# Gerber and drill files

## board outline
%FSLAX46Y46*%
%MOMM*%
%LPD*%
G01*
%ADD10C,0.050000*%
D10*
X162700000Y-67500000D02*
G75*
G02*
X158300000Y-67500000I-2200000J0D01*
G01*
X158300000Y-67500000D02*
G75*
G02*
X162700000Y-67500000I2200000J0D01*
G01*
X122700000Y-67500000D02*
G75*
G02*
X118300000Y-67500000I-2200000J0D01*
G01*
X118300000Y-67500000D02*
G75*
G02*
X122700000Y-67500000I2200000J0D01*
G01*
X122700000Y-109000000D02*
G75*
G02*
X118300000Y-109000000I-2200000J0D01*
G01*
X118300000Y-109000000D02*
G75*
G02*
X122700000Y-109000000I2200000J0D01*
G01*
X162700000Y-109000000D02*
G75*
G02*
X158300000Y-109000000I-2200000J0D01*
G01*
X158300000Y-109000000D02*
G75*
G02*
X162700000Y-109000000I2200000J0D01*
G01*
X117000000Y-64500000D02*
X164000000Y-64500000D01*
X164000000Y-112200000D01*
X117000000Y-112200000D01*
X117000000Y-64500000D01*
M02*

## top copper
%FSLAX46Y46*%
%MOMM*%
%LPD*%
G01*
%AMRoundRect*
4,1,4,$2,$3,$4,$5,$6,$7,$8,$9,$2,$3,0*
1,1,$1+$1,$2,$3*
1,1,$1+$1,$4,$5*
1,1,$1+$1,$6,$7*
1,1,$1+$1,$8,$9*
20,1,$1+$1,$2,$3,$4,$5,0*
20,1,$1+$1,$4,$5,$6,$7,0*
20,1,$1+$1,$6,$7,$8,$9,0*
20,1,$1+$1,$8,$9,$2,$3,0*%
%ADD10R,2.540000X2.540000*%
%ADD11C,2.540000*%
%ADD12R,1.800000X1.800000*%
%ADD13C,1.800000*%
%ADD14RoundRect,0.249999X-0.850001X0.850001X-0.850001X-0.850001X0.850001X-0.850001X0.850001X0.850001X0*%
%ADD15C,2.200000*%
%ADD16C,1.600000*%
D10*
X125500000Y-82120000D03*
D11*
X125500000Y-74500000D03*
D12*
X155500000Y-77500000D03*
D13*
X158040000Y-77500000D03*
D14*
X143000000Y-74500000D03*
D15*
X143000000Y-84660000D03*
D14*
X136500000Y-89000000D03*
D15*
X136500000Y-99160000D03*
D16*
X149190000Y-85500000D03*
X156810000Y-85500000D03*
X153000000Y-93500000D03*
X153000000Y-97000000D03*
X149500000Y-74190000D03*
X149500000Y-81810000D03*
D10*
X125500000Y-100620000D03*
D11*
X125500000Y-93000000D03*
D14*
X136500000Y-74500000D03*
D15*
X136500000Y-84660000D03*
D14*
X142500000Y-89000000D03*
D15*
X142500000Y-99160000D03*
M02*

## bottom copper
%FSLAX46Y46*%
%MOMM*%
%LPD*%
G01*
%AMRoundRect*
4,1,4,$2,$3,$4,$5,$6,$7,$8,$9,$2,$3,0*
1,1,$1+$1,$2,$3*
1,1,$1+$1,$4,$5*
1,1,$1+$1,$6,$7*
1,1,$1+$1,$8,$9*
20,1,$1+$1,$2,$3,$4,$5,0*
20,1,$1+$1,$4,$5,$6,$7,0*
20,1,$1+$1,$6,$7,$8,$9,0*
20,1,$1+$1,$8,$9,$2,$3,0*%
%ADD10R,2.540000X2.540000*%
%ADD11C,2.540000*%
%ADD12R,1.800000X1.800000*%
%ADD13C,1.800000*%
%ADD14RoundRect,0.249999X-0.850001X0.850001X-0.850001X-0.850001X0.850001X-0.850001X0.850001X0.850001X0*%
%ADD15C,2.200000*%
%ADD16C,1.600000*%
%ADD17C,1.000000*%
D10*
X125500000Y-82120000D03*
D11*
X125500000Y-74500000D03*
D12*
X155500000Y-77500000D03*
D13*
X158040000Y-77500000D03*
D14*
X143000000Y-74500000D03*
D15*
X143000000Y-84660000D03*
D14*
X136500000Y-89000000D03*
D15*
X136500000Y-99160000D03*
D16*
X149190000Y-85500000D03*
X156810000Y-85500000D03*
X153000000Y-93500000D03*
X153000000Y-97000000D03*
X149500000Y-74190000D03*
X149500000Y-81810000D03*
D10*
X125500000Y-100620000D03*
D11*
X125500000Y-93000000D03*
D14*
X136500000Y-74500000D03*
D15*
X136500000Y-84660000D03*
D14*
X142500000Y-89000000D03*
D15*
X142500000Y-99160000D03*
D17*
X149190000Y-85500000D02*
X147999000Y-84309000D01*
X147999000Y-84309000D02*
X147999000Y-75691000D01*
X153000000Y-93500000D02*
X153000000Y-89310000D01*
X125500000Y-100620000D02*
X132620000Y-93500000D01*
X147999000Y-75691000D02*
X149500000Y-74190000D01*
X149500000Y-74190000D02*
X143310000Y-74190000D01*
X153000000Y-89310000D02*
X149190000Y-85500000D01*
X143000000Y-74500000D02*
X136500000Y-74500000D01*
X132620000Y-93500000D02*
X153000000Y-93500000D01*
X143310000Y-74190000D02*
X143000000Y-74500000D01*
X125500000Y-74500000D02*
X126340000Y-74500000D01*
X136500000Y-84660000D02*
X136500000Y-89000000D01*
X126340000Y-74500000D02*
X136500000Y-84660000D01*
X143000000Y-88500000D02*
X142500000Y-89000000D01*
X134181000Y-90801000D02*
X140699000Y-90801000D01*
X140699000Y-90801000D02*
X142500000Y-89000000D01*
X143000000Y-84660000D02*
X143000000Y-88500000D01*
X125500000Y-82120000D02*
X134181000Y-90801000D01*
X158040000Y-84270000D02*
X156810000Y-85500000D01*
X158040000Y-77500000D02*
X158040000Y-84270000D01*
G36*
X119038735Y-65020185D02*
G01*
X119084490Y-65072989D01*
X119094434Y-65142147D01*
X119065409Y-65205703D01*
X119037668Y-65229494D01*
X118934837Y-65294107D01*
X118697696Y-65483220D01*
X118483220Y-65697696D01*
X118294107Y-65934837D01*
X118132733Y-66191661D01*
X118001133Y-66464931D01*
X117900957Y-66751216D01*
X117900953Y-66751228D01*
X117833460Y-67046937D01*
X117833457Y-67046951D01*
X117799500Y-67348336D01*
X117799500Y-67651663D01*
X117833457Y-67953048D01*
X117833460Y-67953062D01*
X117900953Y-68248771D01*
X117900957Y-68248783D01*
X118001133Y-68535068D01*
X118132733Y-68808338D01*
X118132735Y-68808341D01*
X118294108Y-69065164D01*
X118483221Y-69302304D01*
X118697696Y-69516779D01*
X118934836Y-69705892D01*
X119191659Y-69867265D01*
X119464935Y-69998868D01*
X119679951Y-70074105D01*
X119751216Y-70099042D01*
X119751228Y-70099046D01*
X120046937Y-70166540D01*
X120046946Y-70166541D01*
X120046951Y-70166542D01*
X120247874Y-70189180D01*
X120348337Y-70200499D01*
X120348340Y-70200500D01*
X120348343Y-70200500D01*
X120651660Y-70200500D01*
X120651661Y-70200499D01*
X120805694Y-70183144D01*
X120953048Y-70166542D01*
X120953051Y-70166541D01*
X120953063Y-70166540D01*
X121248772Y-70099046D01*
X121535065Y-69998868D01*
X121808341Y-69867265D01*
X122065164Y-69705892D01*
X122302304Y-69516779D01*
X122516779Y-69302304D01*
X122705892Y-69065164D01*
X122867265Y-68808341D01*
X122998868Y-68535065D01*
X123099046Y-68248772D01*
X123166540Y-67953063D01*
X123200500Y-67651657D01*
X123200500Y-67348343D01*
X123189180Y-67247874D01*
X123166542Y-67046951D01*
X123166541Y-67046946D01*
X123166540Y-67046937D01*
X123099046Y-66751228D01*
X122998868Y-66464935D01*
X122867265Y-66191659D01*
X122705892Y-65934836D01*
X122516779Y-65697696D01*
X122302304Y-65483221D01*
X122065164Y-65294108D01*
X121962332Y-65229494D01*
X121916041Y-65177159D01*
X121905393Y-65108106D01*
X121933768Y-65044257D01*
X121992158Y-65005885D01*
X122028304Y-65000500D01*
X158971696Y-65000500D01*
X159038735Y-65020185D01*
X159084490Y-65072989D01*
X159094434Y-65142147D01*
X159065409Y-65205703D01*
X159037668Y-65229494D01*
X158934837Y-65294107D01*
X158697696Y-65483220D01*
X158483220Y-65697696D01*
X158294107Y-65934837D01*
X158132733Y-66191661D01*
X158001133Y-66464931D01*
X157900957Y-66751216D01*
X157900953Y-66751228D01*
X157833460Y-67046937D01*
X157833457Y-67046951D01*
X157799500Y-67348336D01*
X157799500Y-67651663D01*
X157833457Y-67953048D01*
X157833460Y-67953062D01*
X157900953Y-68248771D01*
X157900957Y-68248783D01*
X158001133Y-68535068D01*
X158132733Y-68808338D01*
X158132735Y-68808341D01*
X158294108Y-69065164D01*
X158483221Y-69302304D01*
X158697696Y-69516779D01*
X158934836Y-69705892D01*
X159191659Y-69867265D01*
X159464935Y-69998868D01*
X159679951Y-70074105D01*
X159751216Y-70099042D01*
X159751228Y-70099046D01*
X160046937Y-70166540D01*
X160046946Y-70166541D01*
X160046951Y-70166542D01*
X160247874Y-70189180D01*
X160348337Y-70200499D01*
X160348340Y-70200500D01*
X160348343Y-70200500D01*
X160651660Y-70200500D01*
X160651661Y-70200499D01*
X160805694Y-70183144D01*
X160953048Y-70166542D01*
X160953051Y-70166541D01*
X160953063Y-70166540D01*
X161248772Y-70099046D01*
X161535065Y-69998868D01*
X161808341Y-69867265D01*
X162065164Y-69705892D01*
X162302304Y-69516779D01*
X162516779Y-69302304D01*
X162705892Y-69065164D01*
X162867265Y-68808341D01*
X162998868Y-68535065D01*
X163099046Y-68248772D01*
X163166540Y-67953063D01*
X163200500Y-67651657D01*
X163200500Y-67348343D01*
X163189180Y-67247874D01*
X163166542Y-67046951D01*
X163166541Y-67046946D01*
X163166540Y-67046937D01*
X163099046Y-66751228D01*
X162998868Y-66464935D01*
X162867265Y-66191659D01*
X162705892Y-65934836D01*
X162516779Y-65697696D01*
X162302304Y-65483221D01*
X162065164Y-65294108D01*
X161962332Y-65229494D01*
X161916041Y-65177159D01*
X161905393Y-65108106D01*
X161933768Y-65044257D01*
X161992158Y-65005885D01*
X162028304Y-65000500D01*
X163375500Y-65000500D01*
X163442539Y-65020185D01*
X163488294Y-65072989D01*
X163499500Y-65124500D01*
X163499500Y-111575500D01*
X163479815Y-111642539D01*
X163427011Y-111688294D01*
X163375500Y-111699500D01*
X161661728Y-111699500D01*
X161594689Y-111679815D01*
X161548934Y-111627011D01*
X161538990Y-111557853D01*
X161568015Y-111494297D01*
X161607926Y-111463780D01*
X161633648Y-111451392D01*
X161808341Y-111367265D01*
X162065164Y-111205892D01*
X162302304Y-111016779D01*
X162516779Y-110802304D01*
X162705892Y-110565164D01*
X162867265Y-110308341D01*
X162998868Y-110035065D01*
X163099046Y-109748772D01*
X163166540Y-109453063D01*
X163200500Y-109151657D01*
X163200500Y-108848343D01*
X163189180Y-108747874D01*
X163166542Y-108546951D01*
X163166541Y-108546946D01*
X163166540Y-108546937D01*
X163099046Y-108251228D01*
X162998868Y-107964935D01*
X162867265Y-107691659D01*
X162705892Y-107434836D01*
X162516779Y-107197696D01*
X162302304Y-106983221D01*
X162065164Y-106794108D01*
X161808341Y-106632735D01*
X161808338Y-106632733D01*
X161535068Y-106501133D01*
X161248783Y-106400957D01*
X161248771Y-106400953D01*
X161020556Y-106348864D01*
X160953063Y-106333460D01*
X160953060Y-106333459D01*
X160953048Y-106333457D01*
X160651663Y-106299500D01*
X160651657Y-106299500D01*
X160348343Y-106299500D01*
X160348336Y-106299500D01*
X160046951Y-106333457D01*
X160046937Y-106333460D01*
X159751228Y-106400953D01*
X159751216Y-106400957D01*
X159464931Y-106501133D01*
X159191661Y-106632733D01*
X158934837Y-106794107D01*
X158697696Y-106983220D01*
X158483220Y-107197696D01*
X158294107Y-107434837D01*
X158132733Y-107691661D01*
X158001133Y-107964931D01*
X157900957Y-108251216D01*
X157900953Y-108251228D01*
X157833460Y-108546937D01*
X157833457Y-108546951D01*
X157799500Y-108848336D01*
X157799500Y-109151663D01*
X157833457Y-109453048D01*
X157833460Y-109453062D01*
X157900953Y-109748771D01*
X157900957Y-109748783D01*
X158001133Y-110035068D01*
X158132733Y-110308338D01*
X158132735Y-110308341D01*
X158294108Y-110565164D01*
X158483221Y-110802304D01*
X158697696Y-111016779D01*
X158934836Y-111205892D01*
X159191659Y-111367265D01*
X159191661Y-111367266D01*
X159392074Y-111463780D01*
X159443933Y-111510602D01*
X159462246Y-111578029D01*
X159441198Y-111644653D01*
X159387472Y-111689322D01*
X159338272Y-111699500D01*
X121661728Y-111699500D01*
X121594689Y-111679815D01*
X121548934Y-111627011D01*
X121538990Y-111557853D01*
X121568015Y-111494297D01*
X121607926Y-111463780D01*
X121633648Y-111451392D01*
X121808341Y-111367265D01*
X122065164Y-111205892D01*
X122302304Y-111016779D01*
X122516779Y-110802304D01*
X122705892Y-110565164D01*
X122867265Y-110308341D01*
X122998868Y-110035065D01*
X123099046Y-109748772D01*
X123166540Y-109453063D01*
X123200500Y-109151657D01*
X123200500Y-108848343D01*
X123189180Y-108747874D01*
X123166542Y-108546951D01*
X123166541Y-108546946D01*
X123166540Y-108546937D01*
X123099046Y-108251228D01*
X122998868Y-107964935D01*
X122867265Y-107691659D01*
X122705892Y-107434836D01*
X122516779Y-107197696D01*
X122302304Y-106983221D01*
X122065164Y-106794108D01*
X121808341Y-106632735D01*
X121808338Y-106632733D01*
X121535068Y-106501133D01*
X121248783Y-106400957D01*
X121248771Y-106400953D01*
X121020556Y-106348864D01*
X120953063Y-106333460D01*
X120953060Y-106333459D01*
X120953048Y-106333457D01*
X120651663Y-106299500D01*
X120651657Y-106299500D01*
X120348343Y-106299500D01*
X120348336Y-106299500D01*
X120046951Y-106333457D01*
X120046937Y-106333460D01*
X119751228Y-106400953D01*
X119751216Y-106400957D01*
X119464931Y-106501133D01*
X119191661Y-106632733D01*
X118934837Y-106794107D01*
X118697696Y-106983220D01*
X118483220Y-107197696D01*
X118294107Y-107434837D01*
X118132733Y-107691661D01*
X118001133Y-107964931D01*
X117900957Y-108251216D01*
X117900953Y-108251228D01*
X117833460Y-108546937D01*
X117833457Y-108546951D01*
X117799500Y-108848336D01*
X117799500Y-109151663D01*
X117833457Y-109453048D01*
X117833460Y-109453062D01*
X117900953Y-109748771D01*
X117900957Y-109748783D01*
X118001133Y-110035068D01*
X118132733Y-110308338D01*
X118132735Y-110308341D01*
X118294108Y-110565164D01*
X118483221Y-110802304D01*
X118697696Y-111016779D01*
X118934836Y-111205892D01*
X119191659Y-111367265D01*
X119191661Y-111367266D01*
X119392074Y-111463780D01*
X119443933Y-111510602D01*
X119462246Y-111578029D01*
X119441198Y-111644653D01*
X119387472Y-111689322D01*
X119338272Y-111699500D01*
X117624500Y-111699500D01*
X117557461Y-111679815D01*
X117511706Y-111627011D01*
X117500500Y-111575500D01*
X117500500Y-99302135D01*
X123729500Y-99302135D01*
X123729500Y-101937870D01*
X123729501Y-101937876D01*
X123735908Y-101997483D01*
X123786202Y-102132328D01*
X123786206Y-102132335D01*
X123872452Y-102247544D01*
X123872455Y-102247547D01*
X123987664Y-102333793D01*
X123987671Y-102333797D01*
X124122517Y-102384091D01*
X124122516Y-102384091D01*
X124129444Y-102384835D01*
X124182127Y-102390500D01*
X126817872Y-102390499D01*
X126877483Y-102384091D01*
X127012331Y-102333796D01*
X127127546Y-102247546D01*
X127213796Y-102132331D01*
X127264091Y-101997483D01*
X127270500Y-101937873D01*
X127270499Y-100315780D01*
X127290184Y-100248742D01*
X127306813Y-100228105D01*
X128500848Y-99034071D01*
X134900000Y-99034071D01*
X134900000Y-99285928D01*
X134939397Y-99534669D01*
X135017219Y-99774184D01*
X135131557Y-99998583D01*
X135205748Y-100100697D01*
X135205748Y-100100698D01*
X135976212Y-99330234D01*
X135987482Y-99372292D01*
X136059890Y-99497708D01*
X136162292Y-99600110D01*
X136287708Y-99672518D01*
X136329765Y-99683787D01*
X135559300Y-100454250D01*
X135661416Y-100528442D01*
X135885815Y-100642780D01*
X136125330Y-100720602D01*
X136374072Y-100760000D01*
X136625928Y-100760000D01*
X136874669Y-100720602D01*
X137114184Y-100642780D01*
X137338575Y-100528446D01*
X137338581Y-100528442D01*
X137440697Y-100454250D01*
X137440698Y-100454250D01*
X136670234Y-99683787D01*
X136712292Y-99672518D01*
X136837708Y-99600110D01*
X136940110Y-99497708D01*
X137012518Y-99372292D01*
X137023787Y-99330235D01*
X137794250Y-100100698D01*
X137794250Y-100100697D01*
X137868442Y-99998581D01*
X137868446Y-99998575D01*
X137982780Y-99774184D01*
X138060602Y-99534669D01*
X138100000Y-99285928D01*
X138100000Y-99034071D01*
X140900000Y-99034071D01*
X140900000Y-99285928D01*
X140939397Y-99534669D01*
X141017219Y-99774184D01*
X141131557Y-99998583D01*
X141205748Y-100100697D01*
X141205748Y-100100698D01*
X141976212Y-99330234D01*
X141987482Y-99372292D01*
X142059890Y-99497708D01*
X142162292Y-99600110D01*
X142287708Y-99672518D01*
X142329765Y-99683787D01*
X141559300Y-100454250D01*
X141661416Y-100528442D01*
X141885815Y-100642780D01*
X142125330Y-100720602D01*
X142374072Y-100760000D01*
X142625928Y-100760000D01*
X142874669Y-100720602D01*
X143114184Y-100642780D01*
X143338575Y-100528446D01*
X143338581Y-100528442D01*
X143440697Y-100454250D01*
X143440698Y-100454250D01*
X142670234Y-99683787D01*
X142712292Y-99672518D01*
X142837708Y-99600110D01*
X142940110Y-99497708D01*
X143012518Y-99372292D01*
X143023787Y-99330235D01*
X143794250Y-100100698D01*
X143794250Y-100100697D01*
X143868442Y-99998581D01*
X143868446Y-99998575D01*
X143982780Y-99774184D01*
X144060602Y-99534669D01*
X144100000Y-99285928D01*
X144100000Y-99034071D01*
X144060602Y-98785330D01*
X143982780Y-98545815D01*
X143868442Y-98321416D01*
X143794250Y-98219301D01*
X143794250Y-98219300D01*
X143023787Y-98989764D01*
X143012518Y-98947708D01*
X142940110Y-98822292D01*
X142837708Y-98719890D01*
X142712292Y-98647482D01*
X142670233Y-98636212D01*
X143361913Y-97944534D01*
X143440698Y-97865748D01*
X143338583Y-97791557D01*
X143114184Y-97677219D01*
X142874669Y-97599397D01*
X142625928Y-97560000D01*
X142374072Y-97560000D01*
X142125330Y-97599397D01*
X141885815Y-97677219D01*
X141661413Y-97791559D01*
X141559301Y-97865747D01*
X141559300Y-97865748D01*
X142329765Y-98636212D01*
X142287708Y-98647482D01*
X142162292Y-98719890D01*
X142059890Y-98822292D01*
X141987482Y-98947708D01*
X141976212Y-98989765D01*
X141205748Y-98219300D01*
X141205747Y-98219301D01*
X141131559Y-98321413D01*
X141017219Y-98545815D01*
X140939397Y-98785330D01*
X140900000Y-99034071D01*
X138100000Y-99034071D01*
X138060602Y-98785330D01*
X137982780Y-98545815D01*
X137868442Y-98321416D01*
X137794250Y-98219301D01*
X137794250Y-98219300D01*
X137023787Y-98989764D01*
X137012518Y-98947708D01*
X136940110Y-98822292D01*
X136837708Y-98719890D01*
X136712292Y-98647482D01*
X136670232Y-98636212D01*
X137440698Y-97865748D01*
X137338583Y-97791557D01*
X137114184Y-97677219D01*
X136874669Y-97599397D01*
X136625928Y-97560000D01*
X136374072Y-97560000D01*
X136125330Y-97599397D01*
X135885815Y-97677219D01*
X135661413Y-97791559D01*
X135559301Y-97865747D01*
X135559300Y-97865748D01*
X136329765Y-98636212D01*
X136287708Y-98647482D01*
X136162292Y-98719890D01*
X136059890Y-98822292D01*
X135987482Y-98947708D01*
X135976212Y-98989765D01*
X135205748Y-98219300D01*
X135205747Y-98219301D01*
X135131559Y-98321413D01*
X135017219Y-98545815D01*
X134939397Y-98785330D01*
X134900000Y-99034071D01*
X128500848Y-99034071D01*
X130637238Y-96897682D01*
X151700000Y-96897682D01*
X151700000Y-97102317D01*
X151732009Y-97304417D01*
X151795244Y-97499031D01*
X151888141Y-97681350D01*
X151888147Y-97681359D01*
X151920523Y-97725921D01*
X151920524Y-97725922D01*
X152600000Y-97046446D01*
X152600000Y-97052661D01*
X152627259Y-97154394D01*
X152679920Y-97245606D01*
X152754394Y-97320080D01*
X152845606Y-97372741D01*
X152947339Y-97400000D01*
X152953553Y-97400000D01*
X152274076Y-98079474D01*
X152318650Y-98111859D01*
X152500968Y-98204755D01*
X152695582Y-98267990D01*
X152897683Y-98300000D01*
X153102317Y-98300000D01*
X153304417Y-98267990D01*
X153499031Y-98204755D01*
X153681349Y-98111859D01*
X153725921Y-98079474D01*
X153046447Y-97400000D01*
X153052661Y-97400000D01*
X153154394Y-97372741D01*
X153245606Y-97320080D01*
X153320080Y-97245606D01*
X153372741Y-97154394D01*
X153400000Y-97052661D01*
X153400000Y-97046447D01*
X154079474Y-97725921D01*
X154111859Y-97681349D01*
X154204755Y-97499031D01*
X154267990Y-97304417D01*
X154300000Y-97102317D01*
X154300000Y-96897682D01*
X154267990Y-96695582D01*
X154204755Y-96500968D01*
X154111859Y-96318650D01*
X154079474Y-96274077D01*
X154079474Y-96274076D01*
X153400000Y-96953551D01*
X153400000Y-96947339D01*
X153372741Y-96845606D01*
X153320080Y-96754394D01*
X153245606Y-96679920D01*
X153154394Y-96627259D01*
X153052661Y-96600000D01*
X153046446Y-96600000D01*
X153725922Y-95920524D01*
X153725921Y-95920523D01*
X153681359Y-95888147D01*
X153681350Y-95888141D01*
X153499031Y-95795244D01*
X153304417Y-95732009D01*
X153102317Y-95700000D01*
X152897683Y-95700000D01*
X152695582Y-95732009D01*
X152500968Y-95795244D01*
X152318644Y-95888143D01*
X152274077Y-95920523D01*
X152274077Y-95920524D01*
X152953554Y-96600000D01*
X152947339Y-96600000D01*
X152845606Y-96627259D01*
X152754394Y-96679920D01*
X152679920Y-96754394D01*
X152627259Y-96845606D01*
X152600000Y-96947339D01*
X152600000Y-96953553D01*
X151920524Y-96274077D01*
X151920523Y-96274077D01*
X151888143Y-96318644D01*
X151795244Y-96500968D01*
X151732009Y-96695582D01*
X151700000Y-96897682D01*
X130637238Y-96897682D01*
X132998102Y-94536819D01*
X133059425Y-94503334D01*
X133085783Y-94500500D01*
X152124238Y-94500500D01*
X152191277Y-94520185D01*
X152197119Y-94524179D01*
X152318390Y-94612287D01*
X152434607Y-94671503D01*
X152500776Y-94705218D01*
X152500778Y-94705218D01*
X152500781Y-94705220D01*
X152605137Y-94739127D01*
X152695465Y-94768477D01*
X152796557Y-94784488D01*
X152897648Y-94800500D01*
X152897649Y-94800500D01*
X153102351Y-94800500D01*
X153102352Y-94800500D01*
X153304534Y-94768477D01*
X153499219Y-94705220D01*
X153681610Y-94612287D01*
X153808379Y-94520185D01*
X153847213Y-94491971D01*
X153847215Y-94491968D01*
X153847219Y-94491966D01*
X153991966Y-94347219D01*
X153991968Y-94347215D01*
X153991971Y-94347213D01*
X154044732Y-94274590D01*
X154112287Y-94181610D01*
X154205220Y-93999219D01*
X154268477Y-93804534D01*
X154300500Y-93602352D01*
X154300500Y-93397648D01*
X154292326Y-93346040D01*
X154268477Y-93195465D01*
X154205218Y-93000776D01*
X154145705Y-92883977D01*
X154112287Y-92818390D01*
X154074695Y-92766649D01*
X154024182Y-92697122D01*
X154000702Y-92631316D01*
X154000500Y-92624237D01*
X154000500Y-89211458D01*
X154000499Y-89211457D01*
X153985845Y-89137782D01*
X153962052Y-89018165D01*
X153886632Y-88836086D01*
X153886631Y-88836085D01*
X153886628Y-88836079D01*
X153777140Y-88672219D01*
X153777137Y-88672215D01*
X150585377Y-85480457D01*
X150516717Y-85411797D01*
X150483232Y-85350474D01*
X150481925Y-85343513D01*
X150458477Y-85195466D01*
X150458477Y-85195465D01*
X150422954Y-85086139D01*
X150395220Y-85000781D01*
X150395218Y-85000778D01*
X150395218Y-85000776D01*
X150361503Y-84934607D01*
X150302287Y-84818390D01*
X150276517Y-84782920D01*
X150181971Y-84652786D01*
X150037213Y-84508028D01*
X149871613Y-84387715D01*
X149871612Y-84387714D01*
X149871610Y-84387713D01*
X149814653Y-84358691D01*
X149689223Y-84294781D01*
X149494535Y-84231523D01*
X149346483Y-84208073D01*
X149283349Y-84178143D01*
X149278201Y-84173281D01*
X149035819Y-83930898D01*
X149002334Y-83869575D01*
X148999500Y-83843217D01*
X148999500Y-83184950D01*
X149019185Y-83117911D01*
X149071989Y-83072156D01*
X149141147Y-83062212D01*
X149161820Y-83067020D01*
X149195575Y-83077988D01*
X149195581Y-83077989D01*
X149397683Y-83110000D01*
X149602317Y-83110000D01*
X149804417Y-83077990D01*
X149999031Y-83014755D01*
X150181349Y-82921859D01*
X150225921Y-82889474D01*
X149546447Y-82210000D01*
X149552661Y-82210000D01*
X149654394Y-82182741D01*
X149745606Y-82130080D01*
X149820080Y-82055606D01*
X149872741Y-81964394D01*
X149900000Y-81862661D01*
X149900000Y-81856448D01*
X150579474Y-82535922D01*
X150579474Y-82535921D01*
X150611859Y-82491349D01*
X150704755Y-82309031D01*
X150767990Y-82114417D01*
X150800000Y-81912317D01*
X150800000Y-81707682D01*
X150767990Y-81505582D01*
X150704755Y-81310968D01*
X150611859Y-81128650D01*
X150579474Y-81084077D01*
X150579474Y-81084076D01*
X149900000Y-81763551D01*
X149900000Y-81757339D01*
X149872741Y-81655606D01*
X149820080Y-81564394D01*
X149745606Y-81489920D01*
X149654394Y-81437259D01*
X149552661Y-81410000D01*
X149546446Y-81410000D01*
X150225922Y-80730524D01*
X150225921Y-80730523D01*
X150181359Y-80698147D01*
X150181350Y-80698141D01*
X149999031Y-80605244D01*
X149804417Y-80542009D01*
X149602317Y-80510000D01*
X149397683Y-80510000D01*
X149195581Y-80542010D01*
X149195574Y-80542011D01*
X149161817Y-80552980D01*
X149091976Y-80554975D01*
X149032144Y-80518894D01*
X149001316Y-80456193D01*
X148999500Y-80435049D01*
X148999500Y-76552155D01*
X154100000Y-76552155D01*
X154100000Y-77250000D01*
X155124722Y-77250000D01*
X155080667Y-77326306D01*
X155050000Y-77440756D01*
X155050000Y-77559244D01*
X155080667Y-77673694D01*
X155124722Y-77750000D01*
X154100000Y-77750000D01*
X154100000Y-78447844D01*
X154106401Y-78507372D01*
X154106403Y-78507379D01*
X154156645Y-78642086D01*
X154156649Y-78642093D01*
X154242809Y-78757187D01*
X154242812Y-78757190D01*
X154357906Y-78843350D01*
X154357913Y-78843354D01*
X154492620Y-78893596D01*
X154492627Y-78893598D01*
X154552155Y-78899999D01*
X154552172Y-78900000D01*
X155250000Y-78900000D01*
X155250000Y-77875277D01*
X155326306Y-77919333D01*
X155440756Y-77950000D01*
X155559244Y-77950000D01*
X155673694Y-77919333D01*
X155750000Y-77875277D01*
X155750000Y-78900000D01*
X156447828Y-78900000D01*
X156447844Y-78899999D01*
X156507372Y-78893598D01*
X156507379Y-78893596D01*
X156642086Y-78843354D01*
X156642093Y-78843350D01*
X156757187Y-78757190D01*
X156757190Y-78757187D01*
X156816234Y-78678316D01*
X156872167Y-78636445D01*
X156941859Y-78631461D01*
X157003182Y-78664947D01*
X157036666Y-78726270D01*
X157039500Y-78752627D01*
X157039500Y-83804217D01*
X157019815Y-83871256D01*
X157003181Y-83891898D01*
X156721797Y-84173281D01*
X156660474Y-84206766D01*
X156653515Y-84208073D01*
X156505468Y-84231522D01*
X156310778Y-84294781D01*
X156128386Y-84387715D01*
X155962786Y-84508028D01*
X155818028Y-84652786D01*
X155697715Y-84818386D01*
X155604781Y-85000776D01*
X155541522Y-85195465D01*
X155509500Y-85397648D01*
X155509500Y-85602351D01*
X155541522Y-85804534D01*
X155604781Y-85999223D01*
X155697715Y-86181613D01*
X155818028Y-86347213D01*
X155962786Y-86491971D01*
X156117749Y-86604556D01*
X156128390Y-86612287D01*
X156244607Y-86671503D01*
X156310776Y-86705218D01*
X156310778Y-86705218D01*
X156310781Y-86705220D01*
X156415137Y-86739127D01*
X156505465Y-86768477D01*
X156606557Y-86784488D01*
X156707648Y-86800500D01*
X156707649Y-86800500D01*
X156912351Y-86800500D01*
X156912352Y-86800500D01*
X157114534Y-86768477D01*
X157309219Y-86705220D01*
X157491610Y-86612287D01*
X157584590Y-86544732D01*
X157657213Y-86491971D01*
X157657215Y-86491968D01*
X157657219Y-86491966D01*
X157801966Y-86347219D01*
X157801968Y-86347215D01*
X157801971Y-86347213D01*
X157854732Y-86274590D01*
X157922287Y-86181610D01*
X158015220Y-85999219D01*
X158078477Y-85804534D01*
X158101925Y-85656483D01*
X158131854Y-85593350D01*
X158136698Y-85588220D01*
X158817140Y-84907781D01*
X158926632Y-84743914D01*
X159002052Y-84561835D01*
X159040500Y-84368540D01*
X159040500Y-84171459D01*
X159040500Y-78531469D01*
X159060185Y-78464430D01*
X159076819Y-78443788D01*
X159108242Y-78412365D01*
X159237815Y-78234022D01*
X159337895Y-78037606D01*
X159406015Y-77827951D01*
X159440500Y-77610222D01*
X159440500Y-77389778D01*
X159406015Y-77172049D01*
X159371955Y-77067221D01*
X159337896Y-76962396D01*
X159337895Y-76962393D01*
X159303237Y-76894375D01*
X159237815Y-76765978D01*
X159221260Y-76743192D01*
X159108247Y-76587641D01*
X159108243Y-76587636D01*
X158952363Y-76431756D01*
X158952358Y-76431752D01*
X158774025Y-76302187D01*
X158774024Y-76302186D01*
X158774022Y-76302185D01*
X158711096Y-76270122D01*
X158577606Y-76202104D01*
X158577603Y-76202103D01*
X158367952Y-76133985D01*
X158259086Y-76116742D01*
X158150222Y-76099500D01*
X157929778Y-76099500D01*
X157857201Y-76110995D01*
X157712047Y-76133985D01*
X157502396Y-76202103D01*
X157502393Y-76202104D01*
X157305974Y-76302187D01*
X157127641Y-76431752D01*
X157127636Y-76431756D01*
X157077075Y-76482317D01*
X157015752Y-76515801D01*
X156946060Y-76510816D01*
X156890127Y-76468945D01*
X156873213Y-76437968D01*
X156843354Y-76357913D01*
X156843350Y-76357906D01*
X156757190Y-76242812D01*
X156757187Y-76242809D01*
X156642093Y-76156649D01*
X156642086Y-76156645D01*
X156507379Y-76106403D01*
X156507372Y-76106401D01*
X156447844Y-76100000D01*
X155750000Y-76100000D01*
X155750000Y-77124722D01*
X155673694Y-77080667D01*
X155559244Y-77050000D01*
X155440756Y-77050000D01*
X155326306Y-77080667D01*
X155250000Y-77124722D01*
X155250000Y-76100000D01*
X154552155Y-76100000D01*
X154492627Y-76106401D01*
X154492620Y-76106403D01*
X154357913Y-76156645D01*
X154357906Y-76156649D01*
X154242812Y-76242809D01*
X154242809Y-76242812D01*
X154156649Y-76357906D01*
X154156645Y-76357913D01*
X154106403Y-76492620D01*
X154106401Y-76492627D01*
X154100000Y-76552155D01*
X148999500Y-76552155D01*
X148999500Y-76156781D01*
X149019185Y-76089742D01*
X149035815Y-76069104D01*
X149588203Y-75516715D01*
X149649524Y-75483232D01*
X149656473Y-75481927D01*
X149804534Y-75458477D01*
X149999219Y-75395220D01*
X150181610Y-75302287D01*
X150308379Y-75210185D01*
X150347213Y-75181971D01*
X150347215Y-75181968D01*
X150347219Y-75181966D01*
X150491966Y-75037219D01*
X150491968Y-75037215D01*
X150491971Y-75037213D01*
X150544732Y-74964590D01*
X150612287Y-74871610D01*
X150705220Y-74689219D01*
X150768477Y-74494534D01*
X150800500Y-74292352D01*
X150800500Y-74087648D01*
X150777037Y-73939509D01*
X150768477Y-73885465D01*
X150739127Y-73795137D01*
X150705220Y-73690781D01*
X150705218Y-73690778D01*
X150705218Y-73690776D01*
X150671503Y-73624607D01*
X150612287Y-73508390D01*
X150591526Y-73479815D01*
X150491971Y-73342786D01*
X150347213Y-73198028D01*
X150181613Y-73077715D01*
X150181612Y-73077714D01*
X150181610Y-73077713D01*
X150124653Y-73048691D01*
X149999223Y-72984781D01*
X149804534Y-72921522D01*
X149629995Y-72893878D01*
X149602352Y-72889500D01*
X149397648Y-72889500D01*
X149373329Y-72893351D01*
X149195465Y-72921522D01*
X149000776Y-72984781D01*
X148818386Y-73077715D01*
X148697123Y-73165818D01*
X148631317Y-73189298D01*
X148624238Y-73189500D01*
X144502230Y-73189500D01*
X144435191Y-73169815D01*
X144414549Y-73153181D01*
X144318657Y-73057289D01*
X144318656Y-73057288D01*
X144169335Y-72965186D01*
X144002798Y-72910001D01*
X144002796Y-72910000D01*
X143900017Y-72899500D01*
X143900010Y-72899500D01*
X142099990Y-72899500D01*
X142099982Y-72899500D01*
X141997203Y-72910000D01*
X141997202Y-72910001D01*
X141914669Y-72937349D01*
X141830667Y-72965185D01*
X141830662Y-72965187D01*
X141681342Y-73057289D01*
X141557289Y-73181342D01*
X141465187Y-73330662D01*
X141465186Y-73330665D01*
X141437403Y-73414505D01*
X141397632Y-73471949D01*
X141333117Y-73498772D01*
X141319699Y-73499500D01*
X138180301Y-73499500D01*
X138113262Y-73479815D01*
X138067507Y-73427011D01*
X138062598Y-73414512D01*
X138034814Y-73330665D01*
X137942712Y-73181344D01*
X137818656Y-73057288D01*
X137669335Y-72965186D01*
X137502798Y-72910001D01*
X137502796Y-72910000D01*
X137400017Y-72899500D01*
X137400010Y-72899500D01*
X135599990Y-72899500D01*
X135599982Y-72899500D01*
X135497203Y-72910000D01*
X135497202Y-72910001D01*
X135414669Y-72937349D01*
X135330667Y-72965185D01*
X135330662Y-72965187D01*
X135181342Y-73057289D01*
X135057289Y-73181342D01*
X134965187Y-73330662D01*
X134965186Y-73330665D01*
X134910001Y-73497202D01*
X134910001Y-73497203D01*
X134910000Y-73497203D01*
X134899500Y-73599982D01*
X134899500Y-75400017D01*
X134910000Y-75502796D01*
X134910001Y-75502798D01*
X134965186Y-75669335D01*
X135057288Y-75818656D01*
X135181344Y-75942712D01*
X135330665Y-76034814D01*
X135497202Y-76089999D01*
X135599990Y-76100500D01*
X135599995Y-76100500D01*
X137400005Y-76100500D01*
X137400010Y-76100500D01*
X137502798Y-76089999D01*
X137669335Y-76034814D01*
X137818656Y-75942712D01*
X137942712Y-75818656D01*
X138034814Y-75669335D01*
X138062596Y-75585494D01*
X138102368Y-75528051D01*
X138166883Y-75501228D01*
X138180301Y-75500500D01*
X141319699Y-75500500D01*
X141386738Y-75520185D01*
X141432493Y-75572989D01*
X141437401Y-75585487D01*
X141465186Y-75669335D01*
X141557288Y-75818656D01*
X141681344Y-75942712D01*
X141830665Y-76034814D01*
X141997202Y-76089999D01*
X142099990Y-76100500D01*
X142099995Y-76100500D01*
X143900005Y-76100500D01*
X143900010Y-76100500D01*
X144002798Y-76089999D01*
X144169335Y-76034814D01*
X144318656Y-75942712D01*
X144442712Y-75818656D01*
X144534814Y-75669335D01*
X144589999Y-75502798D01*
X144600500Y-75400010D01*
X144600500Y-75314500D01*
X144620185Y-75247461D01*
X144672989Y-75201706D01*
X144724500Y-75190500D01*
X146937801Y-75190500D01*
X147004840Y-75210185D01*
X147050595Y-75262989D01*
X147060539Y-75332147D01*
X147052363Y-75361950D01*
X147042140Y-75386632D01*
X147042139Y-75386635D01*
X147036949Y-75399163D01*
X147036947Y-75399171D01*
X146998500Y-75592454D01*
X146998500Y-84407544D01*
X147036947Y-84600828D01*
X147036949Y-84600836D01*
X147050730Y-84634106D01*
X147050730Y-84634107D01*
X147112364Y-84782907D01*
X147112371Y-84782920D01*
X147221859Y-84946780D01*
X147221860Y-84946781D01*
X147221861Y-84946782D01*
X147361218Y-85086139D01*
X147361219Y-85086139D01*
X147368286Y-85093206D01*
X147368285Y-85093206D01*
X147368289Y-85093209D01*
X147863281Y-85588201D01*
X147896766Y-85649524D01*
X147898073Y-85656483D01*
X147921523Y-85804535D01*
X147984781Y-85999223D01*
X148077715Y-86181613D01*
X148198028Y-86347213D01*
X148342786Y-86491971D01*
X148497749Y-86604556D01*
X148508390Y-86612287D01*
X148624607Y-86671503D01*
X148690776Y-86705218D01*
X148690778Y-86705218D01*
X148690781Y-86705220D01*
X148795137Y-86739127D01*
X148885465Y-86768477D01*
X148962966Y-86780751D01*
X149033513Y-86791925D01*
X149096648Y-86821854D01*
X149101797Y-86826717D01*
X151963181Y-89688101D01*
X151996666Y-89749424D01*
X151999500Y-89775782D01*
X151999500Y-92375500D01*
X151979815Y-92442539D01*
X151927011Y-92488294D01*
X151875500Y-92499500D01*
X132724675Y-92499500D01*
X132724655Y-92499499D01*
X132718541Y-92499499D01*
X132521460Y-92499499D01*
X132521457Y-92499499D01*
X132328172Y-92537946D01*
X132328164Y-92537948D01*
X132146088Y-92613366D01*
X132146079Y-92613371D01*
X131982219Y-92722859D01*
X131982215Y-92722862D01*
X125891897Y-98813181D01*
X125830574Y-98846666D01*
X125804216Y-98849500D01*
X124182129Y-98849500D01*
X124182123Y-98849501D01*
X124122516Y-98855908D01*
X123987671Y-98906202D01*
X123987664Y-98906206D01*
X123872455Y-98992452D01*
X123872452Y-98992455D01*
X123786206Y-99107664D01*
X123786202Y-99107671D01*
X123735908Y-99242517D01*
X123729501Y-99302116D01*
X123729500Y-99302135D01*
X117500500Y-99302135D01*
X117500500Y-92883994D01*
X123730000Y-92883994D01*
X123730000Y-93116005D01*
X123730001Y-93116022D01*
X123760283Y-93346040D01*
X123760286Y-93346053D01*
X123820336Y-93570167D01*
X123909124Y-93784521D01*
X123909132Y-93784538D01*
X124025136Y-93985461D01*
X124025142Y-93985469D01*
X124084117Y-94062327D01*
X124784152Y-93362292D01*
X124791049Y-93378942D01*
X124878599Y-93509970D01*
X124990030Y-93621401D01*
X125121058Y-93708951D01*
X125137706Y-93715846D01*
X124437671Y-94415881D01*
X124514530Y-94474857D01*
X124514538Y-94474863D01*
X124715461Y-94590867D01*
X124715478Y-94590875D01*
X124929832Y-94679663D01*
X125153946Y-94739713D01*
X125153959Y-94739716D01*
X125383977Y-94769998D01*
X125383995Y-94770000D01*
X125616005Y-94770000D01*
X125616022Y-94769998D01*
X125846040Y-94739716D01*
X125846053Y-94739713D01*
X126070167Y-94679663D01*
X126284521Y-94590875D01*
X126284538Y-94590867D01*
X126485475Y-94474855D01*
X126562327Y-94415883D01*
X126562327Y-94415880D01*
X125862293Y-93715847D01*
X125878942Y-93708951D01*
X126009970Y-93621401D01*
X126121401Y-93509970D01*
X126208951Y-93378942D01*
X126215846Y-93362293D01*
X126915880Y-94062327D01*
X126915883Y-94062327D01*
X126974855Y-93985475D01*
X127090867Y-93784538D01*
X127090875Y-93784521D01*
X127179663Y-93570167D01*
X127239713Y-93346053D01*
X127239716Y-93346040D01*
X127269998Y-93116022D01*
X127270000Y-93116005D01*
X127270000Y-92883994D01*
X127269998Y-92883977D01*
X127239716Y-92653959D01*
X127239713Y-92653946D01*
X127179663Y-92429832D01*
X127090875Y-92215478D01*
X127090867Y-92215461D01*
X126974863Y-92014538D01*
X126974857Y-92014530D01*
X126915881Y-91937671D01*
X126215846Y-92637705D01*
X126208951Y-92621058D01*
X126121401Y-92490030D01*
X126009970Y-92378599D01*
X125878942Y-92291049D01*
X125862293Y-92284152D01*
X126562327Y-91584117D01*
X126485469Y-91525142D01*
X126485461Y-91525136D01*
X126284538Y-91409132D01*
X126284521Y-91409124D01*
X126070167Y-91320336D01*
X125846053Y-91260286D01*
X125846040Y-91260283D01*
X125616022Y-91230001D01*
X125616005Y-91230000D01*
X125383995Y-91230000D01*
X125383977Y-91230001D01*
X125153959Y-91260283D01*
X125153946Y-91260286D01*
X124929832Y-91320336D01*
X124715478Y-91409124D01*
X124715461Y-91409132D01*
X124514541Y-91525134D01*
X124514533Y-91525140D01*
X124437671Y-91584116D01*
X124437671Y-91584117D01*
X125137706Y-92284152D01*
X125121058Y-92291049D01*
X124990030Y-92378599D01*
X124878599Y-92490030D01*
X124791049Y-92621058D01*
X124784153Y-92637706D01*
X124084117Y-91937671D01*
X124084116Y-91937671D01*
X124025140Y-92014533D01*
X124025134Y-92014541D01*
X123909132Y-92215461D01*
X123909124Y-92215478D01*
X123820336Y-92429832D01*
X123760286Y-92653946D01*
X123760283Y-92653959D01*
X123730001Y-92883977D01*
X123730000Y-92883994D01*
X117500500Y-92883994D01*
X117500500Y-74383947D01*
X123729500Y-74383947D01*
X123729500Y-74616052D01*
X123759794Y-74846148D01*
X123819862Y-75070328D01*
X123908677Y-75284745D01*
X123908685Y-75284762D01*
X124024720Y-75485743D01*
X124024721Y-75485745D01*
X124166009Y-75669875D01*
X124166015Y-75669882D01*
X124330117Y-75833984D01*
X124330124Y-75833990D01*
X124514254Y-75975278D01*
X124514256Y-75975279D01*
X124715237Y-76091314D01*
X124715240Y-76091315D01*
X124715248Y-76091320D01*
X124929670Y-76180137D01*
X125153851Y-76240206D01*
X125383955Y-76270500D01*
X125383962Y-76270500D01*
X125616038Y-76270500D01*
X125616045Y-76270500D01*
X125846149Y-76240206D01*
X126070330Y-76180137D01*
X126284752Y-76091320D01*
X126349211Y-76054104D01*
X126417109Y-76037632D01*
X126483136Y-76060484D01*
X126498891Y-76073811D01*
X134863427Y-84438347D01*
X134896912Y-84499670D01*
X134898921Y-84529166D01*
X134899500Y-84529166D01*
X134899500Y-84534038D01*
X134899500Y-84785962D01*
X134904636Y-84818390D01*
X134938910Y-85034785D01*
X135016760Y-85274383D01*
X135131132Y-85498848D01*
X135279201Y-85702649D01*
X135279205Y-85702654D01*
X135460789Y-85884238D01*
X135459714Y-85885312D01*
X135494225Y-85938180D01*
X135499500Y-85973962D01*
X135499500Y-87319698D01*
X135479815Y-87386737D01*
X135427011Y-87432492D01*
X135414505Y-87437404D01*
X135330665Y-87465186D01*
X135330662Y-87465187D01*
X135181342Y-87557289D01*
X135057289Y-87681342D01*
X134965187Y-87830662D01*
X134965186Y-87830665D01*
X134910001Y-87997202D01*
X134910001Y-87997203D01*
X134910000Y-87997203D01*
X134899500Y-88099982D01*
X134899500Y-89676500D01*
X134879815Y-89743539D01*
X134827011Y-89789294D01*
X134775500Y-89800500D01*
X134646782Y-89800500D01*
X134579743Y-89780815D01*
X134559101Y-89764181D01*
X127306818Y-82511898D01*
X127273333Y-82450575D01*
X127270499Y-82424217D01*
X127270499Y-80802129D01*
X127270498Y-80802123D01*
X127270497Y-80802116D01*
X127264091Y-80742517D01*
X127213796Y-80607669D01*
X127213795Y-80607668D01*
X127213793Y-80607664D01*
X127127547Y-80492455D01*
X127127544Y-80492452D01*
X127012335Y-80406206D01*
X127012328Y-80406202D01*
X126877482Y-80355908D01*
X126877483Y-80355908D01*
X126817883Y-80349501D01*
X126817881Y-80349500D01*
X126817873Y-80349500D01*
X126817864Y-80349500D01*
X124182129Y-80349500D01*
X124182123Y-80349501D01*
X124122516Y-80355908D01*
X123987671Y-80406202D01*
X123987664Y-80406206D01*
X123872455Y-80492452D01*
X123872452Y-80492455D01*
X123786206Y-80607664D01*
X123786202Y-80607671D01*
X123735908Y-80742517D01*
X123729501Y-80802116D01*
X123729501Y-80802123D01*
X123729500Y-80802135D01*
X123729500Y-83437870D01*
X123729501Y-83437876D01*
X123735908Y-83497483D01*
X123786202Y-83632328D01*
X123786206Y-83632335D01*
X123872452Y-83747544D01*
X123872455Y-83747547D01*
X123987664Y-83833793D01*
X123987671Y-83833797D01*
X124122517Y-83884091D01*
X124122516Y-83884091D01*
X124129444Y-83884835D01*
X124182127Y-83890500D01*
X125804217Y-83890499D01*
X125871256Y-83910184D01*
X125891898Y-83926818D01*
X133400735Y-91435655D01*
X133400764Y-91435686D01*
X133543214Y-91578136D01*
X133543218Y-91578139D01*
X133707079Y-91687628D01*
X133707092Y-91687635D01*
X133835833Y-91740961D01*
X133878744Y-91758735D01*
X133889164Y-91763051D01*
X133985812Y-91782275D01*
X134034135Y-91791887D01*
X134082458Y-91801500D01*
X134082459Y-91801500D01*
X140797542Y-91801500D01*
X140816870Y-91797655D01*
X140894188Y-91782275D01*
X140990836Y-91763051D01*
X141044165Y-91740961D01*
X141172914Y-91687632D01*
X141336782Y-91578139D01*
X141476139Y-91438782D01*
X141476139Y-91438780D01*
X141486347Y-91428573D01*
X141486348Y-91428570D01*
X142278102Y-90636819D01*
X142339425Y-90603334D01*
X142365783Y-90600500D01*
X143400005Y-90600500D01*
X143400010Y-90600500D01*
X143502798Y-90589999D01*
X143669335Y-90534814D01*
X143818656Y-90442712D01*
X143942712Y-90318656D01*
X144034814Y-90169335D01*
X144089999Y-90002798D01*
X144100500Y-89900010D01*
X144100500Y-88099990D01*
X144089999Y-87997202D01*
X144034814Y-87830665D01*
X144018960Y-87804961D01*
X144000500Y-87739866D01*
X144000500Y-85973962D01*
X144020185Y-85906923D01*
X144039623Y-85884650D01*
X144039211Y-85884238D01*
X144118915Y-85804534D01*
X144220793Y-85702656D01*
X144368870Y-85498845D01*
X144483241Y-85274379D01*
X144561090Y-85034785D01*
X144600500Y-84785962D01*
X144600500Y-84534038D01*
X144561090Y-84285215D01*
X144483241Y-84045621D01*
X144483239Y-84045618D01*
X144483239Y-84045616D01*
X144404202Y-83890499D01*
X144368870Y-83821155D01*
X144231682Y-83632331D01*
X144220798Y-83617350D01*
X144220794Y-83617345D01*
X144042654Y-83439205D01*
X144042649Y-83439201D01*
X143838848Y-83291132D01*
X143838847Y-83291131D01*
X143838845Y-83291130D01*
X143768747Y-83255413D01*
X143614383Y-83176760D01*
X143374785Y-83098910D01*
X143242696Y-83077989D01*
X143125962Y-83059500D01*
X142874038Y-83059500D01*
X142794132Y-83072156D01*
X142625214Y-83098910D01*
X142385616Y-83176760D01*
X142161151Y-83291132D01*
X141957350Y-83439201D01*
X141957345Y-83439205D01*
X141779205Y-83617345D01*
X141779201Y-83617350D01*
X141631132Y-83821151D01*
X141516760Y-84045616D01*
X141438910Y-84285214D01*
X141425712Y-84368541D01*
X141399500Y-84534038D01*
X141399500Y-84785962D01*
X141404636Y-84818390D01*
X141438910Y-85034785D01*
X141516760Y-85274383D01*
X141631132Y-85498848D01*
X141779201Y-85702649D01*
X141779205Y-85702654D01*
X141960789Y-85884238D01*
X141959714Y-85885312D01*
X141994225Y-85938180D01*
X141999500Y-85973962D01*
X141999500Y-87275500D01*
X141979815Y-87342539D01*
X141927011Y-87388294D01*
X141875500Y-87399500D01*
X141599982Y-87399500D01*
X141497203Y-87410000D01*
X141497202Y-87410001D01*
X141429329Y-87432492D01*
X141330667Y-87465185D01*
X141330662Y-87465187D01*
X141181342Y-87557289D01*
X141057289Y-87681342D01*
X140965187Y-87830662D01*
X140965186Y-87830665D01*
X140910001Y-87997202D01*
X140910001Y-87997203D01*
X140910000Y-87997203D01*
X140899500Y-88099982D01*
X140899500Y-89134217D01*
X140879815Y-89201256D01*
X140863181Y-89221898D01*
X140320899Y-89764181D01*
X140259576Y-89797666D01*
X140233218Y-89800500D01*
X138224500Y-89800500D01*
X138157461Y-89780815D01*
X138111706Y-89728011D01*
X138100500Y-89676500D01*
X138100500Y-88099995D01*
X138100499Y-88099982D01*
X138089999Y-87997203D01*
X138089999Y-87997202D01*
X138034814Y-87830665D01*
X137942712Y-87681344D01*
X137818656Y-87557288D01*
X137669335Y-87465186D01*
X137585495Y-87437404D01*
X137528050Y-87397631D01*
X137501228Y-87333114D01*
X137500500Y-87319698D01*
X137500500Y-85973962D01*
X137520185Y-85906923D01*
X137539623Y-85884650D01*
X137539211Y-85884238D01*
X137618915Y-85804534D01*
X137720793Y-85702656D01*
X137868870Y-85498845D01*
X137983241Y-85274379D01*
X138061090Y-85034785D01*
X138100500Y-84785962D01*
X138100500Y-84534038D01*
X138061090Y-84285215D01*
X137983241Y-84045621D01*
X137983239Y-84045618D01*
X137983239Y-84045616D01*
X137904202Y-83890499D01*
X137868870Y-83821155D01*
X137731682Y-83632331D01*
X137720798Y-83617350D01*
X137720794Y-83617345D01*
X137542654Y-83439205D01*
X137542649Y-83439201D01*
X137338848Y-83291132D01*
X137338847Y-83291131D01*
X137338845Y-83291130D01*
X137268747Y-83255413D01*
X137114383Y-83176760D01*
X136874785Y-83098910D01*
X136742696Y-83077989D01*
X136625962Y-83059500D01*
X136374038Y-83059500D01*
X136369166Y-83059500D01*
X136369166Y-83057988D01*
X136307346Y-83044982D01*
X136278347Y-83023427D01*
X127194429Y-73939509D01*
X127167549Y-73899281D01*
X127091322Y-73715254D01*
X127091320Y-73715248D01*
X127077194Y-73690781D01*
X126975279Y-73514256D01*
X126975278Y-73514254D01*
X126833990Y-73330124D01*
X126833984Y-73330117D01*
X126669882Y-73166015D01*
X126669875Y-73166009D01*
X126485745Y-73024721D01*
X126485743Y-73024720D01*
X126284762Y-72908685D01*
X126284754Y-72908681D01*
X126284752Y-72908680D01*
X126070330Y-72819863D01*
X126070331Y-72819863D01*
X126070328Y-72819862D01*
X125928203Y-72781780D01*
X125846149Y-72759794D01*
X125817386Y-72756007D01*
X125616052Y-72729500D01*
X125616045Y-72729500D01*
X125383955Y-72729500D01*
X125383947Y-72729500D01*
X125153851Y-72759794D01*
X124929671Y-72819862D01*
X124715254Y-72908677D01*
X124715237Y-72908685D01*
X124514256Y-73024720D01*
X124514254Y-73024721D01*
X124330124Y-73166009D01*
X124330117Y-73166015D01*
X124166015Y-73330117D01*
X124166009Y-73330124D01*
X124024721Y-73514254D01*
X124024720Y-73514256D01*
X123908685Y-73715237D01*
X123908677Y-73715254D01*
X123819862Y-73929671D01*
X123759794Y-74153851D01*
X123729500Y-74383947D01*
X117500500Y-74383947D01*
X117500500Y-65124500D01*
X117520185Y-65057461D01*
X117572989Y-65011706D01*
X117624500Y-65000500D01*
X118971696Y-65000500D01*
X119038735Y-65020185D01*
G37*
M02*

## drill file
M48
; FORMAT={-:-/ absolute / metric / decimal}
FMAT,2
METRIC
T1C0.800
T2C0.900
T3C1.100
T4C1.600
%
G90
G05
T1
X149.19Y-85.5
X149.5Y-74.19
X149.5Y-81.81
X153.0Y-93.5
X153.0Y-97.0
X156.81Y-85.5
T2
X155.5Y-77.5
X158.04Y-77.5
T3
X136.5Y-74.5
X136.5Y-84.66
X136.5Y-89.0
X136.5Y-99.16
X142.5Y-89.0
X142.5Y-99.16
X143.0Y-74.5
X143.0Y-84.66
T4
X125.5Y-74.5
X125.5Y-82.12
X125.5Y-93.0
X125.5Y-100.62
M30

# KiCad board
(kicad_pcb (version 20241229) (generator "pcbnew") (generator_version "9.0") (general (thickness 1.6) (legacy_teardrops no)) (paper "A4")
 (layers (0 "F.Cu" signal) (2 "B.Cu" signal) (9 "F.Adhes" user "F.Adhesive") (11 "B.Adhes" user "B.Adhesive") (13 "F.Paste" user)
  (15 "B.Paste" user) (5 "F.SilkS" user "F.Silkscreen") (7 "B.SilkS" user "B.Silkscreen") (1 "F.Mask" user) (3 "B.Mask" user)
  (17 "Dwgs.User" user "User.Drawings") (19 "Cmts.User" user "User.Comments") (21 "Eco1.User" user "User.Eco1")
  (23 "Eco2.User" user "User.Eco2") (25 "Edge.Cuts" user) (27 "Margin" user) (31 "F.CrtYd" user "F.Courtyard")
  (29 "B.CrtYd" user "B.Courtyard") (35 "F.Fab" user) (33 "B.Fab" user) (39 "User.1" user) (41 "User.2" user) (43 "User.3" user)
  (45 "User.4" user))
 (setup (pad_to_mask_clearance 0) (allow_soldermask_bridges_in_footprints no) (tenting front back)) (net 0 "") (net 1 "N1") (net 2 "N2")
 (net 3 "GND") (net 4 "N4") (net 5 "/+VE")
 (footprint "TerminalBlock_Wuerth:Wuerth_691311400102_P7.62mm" (layer "F.Cu") (at 125.5 82.12 90)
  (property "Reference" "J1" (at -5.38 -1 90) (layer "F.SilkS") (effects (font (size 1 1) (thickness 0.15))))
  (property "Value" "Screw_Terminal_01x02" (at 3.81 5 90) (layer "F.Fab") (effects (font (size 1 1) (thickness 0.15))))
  (pad "1" thru_hole rect (at 0 0 90) (size 2.54 2.54) (drill 1.6) (layers "*.Cu" "*.Mask") (remove_unused_layers no) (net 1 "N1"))
  (pad "2" thru_hole circle (at 7.62 0 90) (size 2.54 2.54) (drill 1.6) (layers "*.Cu" "*.Mask") (remove_unused_layers no) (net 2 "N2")))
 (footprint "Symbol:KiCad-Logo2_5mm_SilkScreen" (layer "F.Cu") (at 147 105.5)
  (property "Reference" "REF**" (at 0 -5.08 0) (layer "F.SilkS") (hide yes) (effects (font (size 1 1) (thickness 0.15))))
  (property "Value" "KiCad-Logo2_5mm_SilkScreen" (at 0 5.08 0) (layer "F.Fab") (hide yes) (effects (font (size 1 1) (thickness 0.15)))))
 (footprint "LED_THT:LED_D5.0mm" (layer "F.Cu") (at 155.5 77.5)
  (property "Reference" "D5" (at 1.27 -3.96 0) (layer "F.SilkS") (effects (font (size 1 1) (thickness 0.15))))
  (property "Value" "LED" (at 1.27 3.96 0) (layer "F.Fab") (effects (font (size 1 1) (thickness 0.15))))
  (pad "1" thru_hole rect (at 0 0) (size 1.8 1.8) (drill 0.9) (layers "*.Cu" "*.Mask") (remove_unused_layers no) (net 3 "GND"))
  (pad "2" thru_hole circle (at 2.54 0) (size 1.8 1.8) (drill 0.9) (layers "*.Cu" "*.Mask") (remove_unused_layers no) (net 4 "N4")))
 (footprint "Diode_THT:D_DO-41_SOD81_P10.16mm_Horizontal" (layer "F.Cu") (at 143 74.5 -90)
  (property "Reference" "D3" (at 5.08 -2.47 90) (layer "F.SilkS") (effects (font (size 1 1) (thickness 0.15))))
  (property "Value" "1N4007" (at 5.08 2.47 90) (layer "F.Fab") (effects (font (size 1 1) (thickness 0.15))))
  (pad "1" thru_hole roundrect (at 0 0 270) (size 2.2 2.2) (drill 1.1) (layers "*.Cu" "*.Mask") (remove_unused_layers no)
   (roundrect_rratio 0.113636) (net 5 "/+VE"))
  (pad "2" thru_hole circle (at 10.16 0 270) (size 2.2 2.2) (drill 1.1) (layers "*.Cu" "*.Mask") (remove_unused_layers no) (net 1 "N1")))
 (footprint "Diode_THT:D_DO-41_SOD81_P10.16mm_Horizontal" (layer "F.Cu") (at 136.5 89 -90)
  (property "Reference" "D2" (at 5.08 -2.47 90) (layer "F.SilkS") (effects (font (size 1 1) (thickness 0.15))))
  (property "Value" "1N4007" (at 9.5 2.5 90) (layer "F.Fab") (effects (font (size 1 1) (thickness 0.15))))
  (pad "1" thru_hole roundrect (at 0 0 270) (size 2.2 2.2) (drill 1.1) (layers "*.Cu" "*.Mask") (remove_unused_layers no)
   (roundrect_rratio 0.113636) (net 2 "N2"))
  (pad "2" thru_hole circle (at 10.16 0 270) (size 2.2 2.2) (drill 1.1) (layers "*.Cu" "*.Mask") (remove_unused_layers no) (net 3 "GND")))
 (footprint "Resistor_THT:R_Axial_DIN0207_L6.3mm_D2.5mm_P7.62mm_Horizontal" (layer "F.Cu") (at 149.19 85.5)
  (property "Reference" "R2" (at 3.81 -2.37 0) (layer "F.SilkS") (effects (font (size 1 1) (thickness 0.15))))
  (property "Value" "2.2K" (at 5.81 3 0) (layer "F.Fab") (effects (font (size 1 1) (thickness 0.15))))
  (pad "1" thru_hole circle (at 0 0) (size 1.6 1.6) (drill 0.8) (layers "*.Cu" "*.Mask") (remove_unused_layers no) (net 5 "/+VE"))
  (pad "2" thru_hole circle (at 7.62 0) (size 1.6 1.6) (drill 0.8) (layers "*.Cu" "*.Mask") (remove_unused_layers no) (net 4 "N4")))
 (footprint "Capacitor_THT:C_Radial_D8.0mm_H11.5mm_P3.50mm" (layer "F.Cu") (at 153 93.5 -90)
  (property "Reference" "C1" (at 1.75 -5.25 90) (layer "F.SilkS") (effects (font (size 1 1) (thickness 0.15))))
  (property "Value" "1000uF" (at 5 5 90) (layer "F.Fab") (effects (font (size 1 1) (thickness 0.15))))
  (pad "1" thru_hole circle (at 0 0 270) (size 1.6 1.6) (drill 0.8) (layers "*.Cu" "*.Mask") (remove_unused_layers no) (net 5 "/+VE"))
  (pad "2" thru_hole circle (at 3.5 0 270) (size 1.6 1.6) (drill 0.8) (layers "*.Cu" "*.Mask") (remove_unused_layers no) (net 3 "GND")))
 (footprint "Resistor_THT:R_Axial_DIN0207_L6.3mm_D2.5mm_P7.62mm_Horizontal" (layer "F.Cu") (at 149.5 74.19 -90)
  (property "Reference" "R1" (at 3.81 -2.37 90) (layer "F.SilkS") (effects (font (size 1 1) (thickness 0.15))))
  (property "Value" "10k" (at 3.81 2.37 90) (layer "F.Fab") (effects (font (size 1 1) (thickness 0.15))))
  (pad "1" thru_hole circle (at 0 0 270) (size 1.6 1.6) (drill 0.8) (layers "*.Cu" "*.Mask") (remove_unused_layers no) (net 5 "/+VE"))
  (pad "2" thru_hole circle (at 7.62 0 270) (size 1.6 1.6) (drill 0.8) (layers "*.Cu" "*.Mask") (remove_unused_layers no) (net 3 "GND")))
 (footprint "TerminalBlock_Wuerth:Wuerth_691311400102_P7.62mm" (layer "F.Cu") (at 125.5 100.62 90)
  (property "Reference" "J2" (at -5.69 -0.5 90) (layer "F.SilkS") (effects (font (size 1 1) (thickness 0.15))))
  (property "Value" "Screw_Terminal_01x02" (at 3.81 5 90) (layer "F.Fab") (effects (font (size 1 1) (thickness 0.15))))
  (pad "1" thru_hole rect (at 0 0 90) (size 2.54 2.54) (drill 1.6) (layers "*.Cu" "*.Mask") (remove_unused_layers no) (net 5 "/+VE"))
  (pad "2" thru_hole circle (at 7.62 0 90) (size 2.54 2.54) (drill 1.6) (layers "*.Cu" "*.Mask") (remove_unused_layers no) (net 3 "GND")))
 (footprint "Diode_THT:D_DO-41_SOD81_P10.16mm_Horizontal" (layer "F.Cu") (at 136.5 74.5 -90)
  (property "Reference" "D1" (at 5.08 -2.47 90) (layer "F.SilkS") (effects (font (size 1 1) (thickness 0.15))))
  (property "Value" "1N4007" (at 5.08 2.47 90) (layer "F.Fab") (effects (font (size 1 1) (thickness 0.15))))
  (pad "1" thru_hole roundrect (at 0 0 270) (size 2.2 2.2) (drill 1.1) (layers "*.Cu" "*.Mask") (remove_unused_layers no)
   (roundrect_rratio 0.113636) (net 5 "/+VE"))
  (pad "2" thru_hole circle (at 10.16 0 270) (size 2.2 2.2) (drill 1.1) (layers "*.Cu" "*.Mask") (remove_unused_layers no) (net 2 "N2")))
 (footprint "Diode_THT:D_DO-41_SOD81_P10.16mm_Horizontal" (layer "F.Cu") (at 142.5 89 -90)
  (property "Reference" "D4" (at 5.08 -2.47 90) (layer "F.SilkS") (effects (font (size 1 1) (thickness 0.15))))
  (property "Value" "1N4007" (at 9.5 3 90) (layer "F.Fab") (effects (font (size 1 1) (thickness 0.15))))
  (pad "1" thru_hole roundrect (at 0 0 270) (size 2.2 2.2) (drill 1.1) (layers "*.Cu" "*.Mask") (remove_unused_layers no)
   (roundrect_rratio 0.113636) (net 1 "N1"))
  (pad "2" thru_hole circle (at 10.16 0 270) (size 2.2 2.2) (drill 1.1) (layers "*.Cu" "*.Mask") (remove_unused_layers no) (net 3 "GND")))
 (gr_circle (center 160.5 67.5) (end 162.7 67.5) (stroke (width 0.05) (type solid)) (fill no) (layer "Edge.Cuts"))
 (gr_circle (center 120.5 67.5) (end 122.7 67.5) (stroke (width 0.05) (type solid)) (fill no) (layer "Edge.Cuts"))
 (gr_circle (center 120.5 109) (end 122.7 109) (stroke (width 0.05) (type solid)) (fill no) (layer "Edge.Cuts"))
 (gr_circle (center 160.5 109) (end 162.7 109) (stroke (width 0.05) (type solid)) (fill no) (layer "Edge.Cuts"))
 (gr_rect (start 117 64.5) (end 164 112.2) (stroke (width 0.05) (type solid)) (fill no) (layer "Edge.Cuts"))
 (segment (start 149.19 85.5) (end 147.999 84.309) (width 1) (layer "B.Cu") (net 5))
 (segment (start 147.999 84.309) (end 147.999 75.691) (width 1) (layer "B.Cu") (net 5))
 (segment (start 153 93.5) (end 153 89.31) (width 1) (layer "B.Cu") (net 5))
 (segment (start 125.5 100.62) (end 132.62 93.5) (width 1) (layer "B.Cu") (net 5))
 (segment (start 147.999 75.691) (end 149.5 74.19) (width 1) (layer "B.Cu") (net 5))
 (segment (start 149.5 74.19) (end 143.31 74.19) (width 1) (layer "B.Cu") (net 5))
 (segment (start 153 89.31) (end 149.19 85.5) (width 1) (layer "B.Cu") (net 5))
 (segment (start 143 74.5) (end 136.5 74.5) (width 1) (layer "B.Cu") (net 5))
 (segment (start 132.62 93.5) (end 153 93.5) (width 1) (layer "B.Cu") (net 5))
 (segment (start 143.31 74.19) (end 143 74.5) (width 1) (layer "B.Cu") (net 5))
 (segment (start 125.5 74.5) (end 126.34 74.5) (width 1) (layer "B.Cu") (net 2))
 (segment (start 136.5 84.66) (end 136.5 89) (width 1) (layer "B.Cu") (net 2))
 (segment (start 126.34 74.5) (end 136.5 84.66) (width 1) (layer "B.Cu") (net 2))
 (segment (start 143 88.5) (end 142.5 89) (width 1) (layer "B.Cu") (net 1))
 (segment (start 134.181 90.801) (end 140.699 90.801) (width 1) (layer "B.Cu") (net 1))
 (segment (start 140.699 90.801) (end 142.5 89) (width 1) (layer "B.Cu") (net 1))
 (segment (start 143 84.66) (end 143 88.5) (width 1) (layer "B.Cu") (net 1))
 (segment (start 125.5 82.12) (end 134.181 90.801) (width 1) (layer "B.Cu") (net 1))
 (segment (start 158.04 84.27) (end 156.81 85.5) (width 1) (layer "B.Cu") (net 4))
 (segment (start 158.04 77.5) (end 158.04 84.27) (width 1) (layer "B.Cu") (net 4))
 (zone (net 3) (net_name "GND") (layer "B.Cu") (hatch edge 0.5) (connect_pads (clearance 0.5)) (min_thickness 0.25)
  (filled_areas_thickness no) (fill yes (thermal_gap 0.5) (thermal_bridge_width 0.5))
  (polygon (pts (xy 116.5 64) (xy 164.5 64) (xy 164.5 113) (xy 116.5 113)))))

